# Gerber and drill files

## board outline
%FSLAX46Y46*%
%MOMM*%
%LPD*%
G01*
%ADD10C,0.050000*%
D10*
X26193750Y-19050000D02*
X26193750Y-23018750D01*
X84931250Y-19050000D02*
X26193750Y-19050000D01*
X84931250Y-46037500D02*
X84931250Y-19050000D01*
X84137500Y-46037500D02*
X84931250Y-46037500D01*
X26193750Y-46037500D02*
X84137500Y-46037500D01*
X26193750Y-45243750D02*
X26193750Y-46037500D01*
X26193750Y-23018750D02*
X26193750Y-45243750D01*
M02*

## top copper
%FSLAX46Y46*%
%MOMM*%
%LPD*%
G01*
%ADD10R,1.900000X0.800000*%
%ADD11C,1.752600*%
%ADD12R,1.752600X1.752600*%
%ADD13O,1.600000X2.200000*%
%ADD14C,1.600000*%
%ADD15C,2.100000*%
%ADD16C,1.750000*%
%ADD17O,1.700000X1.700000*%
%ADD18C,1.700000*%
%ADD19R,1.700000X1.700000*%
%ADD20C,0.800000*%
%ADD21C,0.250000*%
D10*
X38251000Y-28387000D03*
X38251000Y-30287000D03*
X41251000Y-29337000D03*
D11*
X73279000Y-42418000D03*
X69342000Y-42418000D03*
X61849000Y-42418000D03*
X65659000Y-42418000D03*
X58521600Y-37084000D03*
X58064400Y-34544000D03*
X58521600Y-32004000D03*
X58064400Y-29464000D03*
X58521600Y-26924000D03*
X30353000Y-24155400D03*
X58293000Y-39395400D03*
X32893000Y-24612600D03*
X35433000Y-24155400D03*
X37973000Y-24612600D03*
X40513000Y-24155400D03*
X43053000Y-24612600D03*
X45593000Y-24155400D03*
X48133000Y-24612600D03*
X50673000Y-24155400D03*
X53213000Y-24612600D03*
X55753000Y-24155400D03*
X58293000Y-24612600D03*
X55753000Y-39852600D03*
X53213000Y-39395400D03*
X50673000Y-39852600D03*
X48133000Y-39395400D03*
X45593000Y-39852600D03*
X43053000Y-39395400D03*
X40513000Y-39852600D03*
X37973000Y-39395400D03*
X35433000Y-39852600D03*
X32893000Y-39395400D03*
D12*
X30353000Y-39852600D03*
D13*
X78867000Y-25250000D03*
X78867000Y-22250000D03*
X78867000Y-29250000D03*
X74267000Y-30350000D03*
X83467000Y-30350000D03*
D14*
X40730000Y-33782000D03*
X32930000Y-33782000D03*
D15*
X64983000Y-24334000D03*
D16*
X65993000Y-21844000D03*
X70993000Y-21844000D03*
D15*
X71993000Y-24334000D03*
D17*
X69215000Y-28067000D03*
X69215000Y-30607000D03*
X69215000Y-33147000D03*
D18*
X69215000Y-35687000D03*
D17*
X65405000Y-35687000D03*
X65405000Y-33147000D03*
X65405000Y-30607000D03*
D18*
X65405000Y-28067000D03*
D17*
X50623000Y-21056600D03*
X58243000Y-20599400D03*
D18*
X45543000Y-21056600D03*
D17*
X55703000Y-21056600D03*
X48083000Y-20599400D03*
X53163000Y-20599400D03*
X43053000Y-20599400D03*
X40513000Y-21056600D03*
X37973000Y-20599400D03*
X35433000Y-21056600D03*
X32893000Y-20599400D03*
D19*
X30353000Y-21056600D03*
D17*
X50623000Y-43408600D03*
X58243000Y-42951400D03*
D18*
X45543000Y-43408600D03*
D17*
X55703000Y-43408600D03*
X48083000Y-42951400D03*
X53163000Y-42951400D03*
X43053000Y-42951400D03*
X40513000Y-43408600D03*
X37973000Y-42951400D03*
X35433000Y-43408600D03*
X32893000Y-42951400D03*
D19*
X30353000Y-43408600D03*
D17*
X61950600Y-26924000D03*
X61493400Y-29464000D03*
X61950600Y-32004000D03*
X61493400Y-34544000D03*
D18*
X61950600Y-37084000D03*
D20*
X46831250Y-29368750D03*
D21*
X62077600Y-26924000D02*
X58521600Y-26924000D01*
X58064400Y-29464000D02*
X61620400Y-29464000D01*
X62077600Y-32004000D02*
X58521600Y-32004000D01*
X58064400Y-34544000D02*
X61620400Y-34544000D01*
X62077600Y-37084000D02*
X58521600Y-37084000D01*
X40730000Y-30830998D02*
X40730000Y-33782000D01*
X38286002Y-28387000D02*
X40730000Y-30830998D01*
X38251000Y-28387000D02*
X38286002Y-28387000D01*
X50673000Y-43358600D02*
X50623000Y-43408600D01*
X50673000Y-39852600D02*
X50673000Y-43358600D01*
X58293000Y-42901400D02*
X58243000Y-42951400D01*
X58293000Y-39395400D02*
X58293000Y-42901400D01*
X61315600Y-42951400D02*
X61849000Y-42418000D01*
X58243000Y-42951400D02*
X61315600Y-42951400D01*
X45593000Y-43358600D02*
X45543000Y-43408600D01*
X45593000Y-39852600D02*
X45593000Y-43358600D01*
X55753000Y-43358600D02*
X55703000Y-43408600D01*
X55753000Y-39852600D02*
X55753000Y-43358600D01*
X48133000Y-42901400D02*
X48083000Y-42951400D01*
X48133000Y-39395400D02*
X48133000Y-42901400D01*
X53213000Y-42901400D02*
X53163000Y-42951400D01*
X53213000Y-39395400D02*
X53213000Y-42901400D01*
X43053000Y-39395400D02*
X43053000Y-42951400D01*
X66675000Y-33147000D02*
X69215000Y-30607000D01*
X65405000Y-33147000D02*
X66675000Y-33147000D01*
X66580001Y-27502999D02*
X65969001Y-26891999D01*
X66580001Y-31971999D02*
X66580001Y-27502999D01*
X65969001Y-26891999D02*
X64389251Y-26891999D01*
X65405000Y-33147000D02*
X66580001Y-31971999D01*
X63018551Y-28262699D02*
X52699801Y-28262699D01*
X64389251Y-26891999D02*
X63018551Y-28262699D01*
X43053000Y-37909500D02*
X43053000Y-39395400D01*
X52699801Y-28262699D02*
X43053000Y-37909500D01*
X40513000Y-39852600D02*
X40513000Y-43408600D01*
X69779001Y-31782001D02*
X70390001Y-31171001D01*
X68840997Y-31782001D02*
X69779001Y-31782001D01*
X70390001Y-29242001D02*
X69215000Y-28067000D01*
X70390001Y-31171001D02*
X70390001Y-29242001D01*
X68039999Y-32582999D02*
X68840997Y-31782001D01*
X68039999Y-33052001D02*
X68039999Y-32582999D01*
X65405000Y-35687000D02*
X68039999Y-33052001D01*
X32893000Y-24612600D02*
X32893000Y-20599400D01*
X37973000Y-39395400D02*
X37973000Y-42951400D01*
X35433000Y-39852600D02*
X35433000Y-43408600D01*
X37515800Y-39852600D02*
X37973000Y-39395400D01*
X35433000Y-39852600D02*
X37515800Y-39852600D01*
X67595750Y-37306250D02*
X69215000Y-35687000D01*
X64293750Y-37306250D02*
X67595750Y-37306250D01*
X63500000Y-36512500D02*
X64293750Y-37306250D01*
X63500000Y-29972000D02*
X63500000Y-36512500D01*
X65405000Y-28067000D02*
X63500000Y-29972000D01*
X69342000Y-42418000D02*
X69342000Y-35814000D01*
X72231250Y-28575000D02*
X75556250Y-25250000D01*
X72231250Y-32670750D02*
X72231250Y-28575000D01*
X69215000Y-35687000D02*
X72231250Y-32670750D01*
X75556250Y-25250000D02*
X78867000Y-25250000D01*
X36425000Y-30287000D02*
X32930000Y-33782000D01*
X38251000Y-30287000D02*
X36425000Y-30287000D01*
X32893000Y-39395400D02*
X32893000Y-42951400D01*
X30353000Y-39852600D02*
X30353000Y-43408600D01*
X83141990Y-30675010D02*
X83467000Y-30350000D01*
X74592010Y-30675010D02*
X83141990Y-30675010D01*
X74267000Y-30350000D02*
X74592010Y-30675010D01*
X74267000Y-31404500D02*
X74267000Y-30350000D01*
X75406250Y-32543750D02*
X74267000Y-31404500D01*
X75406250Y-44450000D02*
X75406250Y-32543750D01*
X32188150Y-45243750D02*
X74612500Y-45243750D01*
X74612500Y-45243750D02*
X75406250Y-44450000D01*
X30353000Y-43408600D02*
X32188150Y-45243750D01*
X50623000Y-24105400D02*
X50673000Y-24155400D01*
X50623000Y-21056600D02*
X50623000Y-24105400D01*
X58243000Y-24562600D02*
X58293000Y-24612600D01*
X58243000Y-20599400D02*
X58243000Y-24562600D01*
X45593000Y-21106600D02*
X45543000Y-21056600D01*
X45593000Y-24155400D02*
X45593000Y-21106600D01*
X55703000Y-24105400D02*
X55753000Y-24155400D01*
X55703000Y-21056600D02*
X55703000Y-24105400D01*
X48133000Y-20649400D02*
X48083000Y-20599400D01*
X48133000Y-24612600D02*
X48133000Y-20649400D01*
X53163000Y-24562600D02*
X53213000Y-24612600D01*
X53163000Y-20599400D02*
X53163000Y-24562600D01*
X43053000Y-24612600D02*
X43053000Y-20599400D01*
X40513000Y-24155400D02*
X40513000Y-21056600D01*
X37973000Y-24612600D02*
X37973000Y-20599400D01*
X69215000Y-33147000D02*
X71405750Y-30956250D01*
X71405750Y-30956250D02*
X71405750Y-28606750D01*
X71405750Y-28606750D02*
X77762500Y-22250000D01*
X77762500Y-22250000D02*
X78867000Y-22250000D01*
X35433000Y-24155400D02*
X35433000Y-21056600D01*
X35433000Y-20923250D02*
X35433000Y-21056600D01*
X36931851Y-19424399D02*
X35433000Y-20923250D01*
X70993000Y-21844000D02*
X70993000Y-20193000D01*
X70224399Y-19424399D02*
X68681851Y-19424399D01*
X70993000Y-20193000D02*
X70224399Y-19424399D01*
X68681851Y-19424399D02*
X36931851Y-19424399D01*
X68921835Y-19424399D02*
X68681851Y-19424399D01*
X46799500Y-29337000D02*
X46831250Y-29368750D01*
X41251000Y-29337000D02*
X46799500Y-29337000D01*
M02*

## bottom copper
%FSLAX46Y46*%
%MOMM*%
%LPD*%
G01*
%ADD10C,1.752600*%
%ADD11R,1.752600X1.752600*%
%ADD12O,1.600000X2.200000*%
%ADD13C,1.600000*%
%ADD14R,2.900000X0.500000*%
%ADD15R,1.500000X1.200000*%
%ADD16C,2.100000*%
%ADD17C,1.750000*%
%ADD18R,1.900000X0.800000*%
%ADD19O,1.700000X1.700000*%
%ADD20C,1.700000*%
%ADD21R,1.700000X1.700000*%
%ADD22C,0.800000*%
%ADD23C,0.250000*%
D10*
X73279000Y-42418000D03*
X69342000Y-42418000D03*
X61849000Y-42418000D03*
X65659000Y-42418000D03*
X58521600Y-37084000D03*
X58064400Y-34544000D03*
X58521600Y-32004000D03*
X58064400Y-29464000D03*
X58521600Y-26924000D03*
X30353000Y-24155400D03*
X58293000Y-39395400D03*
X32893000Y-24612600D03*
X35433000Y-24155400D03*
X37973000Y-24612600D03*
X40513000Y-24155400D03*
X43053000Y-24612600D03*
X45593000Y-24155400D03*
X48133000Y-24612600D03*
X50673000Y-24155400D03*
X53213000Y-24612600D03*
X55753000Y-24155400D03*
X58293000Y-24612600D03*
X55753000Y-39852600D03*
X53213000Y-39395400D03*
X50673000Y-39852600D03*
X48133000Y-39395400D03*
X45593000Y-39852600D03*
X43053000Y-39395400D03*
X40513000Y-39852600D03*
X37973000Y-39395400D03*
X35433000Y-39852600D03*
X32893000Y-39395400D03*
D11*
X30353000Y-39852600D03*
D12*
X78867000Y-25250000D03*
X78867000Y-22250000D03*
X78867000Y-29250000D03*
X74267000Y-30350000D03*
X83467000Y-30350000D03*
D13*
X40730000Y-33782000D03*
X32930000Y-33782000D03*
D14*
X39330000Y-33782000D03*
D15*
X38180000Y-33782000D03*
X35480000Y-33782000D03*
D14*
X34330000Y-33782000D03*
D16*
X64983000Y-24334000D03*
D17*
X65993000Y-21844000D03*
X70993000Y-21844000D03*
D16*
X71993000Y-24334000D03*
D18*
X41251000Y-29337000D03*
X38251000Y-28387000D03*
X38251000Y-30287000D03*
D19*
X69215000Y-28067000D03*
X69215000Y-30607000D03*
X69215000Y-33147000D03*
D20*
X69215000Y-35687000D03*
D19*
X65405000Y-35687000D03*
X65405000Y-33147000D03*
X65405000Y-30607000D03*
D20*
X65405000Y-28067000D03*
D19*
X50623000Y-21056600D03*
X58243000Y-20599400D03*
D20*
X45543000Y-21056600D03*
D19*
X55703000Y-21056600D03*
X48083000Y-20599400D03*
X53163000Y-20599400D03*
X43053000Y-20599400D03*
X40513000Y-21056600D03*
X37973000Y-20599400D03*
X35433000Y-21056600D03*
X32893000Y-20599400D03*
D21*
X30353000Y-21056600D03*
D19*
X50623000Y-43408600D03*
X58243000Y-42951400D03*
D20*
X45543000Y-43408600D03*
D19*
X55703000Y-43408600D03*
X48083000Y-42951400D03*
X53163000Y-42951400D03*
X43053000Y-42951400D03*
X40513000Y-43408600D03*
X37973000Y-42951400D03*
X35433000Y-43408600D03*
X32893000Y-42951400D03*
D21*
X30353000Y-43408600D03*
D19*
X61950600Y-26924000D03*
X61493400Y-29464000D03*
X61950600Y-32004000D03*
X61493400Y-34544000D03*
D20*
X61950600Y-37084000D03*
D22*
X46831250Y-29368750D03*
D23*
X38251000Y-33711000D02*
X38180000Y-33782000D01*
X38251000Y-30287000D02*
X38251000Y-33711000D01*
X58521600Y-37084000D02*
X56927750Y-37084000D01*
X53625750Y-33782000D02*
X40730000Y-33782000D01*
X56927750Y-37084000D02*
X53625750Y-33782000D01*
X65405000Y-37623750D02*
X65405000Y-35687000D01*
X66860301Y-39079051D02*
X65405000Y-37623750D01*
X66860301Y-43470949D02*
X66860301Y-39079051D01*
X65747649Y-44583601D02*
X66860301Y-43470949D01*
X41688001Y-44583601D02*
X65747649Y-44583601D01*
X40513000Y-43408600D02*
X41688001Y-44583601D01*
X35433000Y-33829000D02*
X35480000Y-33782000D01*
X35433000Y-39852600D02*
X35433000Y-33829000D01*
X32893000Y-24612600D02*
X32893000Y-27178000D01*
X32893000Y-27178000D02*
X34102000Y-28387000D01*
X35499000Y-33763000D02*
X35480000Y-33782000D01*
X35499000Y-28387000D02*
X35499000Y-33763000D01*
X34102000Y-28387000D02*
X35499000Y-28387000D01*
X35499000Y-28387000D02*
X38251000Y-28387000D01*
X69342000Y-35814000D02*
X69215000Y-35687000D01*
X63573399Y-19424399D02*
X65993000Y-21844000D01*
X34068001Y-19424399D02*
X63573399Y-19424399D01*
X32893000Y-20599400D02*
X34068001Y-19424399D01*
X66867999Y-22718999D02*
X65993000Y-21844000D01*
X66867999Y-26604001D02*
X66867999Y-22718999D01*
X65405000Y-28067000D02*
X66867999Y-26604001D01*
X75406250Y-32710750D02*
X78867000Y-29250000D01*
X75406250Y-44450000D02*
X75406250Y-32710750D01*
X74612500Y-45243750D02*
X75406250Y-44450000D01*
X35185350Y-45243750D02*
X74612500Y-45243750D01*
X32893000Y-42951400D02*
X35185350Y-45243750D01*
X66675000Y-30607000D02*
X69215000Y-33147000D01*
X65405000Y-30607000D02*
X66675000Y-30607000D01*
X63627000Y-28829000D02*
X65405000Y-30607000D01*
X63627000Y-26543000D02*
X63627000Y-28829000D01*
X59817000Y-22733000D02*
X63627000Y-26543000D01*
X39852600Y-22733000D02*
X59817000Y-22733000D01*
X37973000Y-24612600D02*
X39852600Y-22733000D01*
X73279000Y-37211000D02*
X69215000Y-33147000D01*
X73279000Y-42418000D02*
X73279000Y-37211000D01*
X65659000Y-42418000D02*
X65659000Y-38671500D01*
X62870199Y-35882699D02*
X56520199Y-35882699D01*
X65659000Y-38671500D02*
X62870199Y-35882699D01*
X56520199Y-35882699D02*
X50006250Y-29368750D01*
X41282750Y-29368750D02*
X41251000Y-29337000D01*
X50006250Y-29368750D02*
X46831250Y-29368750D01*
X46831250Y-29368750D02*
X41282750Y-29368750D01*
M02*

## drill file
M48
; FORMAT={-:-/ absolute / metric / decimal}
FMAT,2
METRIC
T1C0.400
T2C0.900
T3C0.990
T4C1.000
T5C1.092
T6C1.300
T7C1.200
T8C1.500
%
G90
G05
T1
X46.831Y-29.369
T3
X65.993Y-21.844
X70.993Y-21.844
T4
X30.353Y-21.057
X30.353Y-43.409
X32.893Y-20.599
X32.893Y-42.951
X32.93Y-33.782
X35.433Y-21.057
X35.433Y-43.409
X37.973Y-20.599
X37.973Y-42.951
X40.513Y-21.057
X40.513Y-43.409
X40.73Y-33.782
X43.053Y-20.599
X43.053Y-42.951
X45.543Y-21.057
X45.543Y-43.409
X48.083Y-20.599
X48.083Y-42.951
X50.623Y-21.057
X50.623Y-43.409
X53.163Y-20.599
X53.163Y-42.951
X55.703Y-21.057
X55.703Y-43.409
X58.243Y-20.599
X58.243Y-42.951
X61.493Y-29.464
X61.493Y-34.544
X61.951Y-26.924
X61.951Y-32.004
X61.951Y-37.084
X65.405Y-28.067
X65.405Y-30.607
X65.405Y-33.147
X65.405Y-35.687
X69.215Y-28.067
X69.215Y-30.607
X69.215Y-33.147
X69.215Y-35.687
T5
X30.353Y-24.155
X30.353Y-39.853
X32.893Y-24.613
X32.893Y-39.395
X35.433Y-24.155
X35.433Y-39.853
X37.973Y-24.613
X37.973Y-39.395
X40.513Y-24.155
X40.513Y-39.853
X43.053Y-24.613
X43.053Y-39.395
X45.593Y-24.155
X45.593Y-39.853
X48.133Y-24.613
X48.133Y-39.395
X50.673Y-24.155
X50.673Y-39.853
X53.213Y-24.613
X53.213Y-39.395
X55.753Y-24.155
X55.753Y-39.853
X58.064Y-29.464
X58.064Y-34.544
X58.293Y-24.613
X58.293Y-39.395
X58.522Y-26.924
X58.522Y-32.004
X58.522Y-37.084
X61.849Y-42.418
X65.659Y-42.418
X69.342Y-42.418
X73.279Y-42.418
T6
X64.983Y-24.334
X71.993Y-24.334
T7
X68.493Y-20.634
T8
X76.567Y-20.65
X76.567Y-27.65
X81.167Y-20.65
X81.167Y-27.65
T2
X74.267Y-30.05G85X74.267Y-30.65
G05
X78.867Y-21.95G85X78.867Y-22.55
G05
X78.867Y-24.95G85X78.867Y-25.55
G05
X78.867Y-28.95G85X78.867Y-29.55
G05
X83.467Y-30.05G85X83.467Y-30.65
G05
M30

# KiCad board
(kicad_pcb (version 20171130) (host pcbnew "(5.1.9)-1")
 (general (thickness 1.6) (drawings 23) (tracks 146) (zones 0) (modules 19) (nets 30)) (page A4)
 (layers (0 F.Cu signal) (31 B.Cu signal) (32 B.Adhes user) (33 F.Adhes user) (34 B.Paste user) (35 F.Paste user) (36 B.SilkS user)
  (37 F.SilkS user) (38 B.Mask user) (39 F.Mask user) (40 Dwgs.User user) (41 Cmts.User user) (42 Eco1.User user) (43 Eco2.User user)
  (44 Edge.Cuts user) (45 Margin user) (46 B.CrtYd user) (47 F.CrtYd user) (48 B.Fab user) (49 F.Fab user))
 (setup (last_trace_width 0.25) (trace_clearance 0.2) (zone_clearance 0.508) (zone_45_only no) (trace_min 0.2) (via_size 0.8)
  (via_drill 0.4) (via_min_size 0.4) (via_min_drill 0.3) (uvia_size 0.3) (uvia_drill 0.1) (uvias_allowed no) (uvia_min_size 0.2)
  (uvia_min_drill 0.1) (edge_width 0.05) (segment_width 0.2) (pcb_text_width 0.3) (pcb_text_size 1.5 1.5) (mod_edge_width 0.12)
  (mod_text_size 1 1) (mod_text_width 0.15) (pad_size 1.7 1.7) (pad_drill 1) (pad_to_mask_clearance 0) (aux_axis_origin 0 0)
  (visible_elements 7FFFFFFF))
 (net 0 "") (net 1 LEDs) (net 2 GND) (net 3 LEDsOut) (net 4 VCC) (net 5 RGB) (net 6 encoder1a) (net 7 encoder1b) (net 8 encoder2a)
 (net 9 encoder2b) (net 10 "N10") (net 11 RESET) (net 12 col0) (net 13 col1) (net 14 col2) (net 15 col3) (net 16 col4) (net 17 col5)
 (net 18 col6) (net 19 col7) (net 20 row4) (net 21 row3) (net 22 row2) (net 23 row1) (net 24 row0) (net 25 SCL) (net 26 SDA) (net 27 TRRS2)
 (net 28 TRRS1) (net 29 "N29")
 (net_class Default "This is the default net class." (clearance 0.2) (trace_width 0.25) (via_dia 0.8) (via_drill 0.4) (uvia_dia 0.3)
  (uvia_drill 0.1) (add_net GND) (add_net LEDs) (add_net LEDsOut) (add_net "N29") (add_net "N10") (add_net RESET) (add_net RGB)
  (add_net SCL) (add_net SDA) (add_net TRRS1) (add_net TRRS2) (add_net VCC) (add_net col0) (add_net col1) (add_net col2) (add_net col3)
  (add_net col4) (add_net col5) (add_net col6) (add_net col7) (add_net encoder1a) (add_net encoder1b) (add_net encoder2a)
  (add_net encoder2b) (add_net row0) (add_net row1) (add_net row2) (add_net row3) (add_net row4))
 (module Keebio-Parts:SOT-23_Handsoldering (layer F.Cu) (at 39.751 29.337)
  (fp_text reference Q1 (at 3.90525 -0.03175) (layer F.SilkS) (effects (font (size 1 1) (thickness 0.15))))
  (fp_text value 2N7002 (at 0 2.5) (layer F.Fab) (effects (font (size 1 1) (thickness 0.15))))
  (pad 1 smd rect (at -1.5 -0.95) (size 1.9 0.8) (layers F.Cu F.Paste F.Mask) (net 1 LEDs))
  (pad 2 smd rect (at -1.5 0.95) (size 1.9 0.8) (layers F.Cu F.Paste F.Mask) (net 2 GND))
  (pad 3 smd rect (at 1.5 0) (size 1.9 0.8) (layers F.Cu F.Paste F.Mask) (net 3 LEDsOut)))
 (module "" (layer F.Cu) (at 73.914 49.149)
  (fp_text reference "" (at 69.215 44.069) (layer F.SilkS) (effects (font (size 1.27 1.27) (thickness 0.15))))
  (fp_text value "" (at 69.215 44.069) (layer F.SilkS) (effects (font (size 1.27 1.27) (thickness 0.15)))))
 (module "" (layer F.Cu) (at 69.215 44.069)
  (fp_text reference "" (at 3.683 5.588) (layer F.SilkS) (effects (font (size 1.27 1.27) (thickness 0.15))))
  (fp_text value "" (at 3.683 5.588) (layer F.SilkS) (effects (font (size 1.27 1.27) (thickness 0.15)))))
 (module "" (layer F.Cu) (at 3.683 5.588)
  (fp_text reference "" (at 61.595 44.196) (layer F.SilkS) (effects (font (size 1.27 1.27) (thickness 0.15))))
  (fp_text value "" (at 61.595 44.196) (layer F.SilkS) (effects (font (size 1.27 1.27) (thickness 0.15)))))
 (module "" (layer F.Cu) (at 61.595 44.196)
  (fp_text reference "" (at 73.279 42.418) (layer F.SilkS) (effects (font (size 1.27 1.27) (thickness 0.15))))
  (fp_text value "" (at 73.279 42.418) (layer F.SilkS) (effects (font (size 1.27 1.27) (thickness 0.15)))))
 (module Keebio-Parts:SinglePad (layer F.Cu) (at 73.279 42.418)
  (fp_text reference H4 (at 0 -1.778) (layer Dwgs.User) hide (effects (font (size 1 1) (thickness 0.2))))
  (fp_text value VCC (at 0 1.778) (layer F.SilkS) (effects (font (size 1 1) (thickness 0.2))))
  (pad 1 thru_hole circle (at 0 0 270) (size 1.7526 1.7526) (drill 1.0922) (layers *.Cu *.SilkS *.Mask) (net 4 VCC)))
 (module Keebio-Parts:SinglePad (layer F.Cu) (at 69.342 42.418)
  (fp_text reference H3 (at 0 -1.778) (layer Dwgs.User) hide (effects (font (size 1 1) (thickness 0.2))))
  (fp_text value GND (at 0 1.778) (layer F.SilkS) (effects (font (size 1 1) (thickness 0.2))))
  (pad 1 thru_hole circle (at 0 0 270) (size 1.7526 1.7526) (drill 1.0922) (layers *.Cu *.SilkS *.Mask) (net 2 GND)))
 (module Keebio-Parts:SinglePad (layer F.Cu) (at 61.849 42.418)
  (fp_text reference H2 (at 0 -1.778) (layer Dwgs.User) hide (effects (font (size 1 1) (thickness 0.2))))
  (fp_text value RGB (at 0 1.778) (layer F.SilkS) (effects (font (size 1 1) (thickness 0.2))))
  (pad 1 thru_hole circle (at 0 0 270) (size 1.7526 1.7526) (drill 1.0922) (layers *.Cu *.SilkS *.Mask) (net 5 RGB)))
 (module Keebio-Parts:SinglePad (layer F.Cu) (at 65.659 42.418)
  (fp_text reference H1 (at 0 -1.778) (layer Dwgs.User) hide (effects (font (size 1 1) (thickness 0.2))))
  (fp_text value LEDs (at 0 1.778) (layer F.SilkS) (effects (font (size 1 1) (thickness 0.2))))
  (pad 1 thru_hole circle (at 0 0 270) (size 1.7526 1.7526) (drill 1.0922) (layers *.Cu *.SilkS *.Mask) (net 3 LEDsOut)))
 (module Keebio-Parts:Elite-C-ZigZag (layer F.Cu) (at 44.323 32.004)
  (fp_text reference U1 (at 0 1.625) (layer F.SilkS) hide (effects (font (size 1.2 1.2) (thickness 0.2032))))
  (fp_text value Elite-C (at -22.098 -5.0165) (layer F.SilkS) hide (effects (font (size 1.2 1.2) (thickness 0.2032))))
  (pad 25 thru_hole circle (at 14.1986 5.08) (size 1.7526 1.7526) (drill 1.0922) (layers *.Cu *.SilkS *.Mask) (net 1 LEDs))
  (pad 26 thru_hole circle (at 13.7414 2.54) (size 1.7526 1.7526) (drill 1.0922) (layers *.Cu *.SilkS *.Mask) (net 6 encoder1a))
  (pad 27 thru_hole circle (at 14.1986 0) (size 1.7526 1.7526) (drill 1.0922) (layers *.Cu *.SilkS *.Mask) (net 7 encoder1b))
  (pad 28 thru_hole circle (at 13.7414 -2.54) (size 1.7526 1.7526) (drill 1.0922) (layers *.Cu *.SilkS *.Mask) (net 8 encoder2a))
  (pad 29 thru_hole circle (at 14.1986 -5.08) (size 1.7526 1.7526) (drill 1.0922) (layers *.Cu *.SilkS *.Mask) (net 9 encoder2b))
  (pad 24 thru_hole circle (at -13.97 -7.8486) (size 1.7526 1.7526) (drill 1.0922) (layers *.Cu *.SilkS *.Mask) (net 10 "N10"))
  (pad 12 thru_hole circle (at 13.97 7.3914) (size 1.7526 1.7526) (drill 1.0922) (layers *.Cu *.SilkS *.Mask) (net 5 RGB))
  (pad 23 thru_hole circle (at -11.43 -7.3914) (size 1.7526 1.7526) (drill 1.0922) (layers *.Cu *.SilkS *.Mask) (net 2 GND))
  (pad 22 thru_hole circle (at -8.89 -7.8486) (size 1.7526 1.7526) (drill 1.0922) (layers *.Cu *.SilkS *.Mask) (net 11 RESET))
  (pad 21 thru_hole circle (at -6.35 -7.3914) (size 1.7526 1.7526) (drill 1.0922) (layers *.Cu *.SilkS *.Mask) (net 4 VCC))
  (pad 20 thru_hole circle (at -3.81 -7.8486) (size 1.7526 1.7526) (drill 1.0922) (layers *.Cu *.SilkS *.Mask) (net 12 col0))
  (pad 19 thru_hole circle (at -1.27 -7.3914) (size 1.7526 1.7526) (drill 1.0922) (layers *.Cu *.SilkS *.Mask) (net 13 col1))
  (pad 18 thru_hole circle (at 1.27 -7.8486) (size 1.7526 1.7526) (drill 1.0922) (layers *.Cu *.SilkS *.Mask) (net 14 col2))
  (pad 17 thru_hole circle (at 3.81 -7.3914) (size 1.7526 1.7526) (drill 1.0922) (layers *.Cu *.SilkS *.Mask) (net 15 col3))
  (pad 16 thru_hole circle (at 6.35 -7.8486) (size 1.7526 1.7526) (drill 1.0922) (layers *.Cu *.SilkS *.Mask) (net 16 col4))
  (pad 15 thru_hole circle (at 8.89 -7.3914) (size 1.7526 1.7526) (drill 1.0922) (layers *.Cu *.SilkS *.Mask) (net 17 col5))
  (pad 14 thru_hole circle (at 11.43 -7.8486) (size 1.7526 1.7526) (drill 1.0922) (layers *.Cu *.SilkS *.Mask) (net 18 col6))
  (pad 13 thru_hole circle (at 13.97 -7.3914) (size 1.7526 1.7526) (drill 1.0922) (layers *.Cu *.SilkS *.Mask) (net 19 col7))
  (pad 11 thru_hole circle (at 11.43 7.8486) (size 1.7526 1.7526) (drill 1.0922) (layers *.Cu *.SilkS *.Mask) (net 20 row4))
  (pad 10 thru_hole circle (at 8.89 7.3914) (size 1.7526 1.7526) (drill 1.0922) (layers *.Cu *.SilkS *.Mask) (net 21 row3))
  (pad 9 thru_hole circle (at 6.35 7.8486) (size 1.7526 1.7526) (drill 1.0922) (layers *.Cu *.SilkS *.Mask) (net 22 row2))
  (pad 8 thru_hole circle (at 3.81 7.3914) (size 1.7526 1.7526) (drill 1.0922) (layers *.Cu *.SilkS *.Mask) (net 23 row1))
  (pad 7 thru_hole circle (at 1.27 7.8486) (size 1.7526 1.7526) (drill 1.0922) (layers *.Cu *.SilkS *.Mask) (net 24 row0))
  (pad 6 thru_hole circle (at -1.27 7.3914) (size 1.7526 1.7526) (drill 1.0922) (layers *.Cu *.SilkS *.Mask) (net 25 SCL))
  (pad 5 thru_hole circle (at -3.81 7.8486) (size 1.7526 1.7526) (drill 1.0922) (layers *.Cu *.SilkS *.Mask) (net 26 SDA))
  (pad 4 thru_hole circle (at -6.35 7.3914) (size 1.7526 1.7526) (drill 1.0922) (layers *.Cu *.SilkS *.Mask) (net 2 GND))
  (pad 3 thru_hole circle (at -8.89 7.8486) (size 1.7526 1.7526) (drill 1.0922) (layers *.Cu *.SilkS *.Mask) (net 2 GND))
  (pad 2 thru_hole circle (at -11.43 7.3914) (size 1.7526 1.7526) (drill 1.0922) (layers *.Cu *.SilkS *.Mask) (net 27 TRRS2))
  (pad 1 thru_hole rect (at -13.97 7.8486) (size 1.7526 1.7526) (drill 1.0922) (layers *.Cu *.SilkS *.Mask) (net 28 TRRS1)))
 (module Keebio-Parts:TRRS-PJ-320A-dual (layer F.Cu) (at 78.867 19.05)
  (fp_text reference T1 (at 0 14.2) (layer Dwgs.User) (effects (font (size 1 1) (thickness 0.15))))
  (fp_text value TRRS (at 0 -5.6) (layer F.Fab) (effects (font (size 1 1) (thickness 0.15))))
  (pad 3 thru_hole oval (at 0 6.2) (size 1.6 2.2) (drill oval 0.9 1.5) (layers *.Cu *.Mask) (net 2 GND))
  (pad "" np_thru_hole circle (at -2.3 1.6) (size 1.5 1.5) (drill 1.5) (layers *.Cu *.Mask))
  (pad "" np_thru_hole circle (at -2.3 8.6) (size 1.5 1.5) (drill 1.5) (layers *.Cu *.Mask))
  (pad 4 thru_hole oval (at 0 3.2) (size 1.6 2.2) (drill oval 0.9 1.5) (layers *.Cu *.Mask) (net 4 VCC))
  (pad 2 thru_hole oval (at 0 10.2) (size 1.6 2.2) (drill oval 0.9 1.5) (layers *.Cu *.Mask) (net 27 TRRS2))
  (pad 1 thru_hole oval (at -4.6 11.3) (size 1.6 2.2) (drill oval 0.9 1.5) (layers *.Cu *.Mask) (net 28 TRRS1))
  (pad 1 thru_hole oval (at 4.6 11.3) (size 1.6 2.2) (drill oval 0.9 1.5) (layers *.Cu *.Mask) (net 28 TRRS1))
  (pad "" np_thru_hole circle (at 2.3 1.6) (size 1.5 1.5) (drill 1.5) (layers *.Cu *.Mask))
  (pad "" np_thru_hole circle (at 2.3 8.6) (size 1.5 1.5) (drill 1.5) (layers *.Cu *.Mask)))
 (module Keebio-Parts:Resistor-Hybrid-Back (layer F.Cu) (at 36.83 33.782)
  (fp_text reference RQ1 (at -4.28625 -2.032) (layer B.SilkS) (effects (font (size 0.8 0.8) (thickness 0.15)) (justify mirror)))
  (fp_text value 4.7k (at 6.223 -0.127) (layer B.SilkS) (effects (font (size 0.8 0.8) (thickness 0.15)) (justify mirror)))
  (pad 1 thru_hole circle (at 3.9 0) (size 1.6 1.6) (drill 1) (layers *.Cu *.Mask) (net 1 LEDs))
  (pad 2 thru_hole circle (at -3.9 0) (size 1.6 1.6) (drill 1) (layers *.Cu *.Mask F.SilkS) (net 2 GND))
  (pad 1 smd rect (at 2.5 0) (size 2.9 0.5) (layers B.Cu) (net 1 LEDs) (solder_mask_margin -999))
  (pad 1 smd rect (at 1.35 0) (size 1.5 1.2) (layers B.Cu B.Paste B.Mask) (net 1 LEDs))
  (pad 2 smd rect (at -1.35 0) (size 1.5 1.2) (layers B.Cu B.Paste B.Mask) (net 2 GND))
  (pad 2 smd rect (at -2.5 0) (size 2.9 0.5) (layers B.Cu) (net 2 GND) (solder_mask_margin -999)))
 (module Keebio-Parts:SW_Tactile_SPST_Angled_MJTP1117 (layer B.Cu) (at 70.993 21.844 180)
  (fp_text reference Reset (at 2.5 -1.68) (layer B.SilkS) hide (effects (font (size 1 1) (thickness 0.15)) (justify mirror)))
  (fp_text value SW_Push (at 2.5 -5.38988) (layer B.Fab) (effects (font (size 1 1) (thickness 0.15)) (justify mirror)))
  (pad "" thru_hole circle (at 6.01 -2.49 180) (size 2.1 2.1) (drill 1.3) (layers *.Cu *.Mask))
  (pad 2 thru_hole circle (at 5 0 180) (size 1.75 1.75) (drill 0.99) (layers *.Cu *.Mask) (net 2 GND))
  (pad 1 thru_hole circle (at 0 0 180) (size 1.75 1.75) (drill 0.99) (layers *.Cu *.Mask) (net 11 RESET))
  (pad "" thru_hole circle (at -1 -2.49 180) (size 2.1 2.1) (drill 1.3) (layers *.Cu *.Mask))
  (pad "" np_thru_hole circle (at 2.5 1.21 180) (size 1.2 1.2) (drill 1.2) (layers *.Cu *.Mask)))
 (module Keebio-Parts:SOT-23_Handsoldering (layer B.Cu) (at 39.751 29.337)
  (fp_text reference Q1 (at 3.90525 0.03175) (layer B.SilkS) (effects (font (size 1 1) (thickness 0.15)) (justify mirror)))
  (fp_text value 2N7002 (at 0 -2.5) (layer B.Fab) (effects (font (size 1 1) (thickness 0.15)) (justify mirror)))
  (pad 3 smd rect (at 1.5 0) (size 1.9 0.8) (layers B.Cu B.Paste B.Mask) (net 3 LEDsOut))
  (pad 2 smd rect (at -1.5 -0.95) (size 1.9 0.8) (layers B.Cu B.Paste B.Mask) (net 2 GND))
  (pad 1 smd rect (at -1.5 0.95) (size 1.9 0.8) (layers B.Cu B.Paste B.Mask) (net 1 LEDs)))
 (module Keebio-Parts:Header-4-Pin (layer F.Cu) (at 69.215 35.687 180)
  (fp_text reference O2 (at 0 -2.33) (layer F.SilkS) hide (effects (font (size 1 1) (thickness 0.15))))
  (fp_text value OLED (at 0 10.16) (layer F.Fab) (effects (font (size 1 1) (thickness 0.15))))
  (pad 4 thru_hole oval (at 0 7.62 180) (size 1.7 1.7) (drill 1) (layers *.Cu *.Mask) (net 26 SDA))
  (pad 3 thru_hole oval (at 0 5.08 180) (size 1.7 1.7) (drill 1) (layers *.Cu *.Mask) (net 25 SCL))
  (pad 2 thru_hole oval (at 0 2.54 180) (size 1.7 1.7) (drill 1) (layers *.Cu *.Mask) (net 4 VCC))
  (pad 1 thru_hole circle (at 0 0 180) (size 1.7 1.7) (drill 1) (layers *.Cu *.Mask) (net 2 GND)))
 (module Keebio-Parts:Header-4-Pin (layer F.Cu) (at 65.405 28.067)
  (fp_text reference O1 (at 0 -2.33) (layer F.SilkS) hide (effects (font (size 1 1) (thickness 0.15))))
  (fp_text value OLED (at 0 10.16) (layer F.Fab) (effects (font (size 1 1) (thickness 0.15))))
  (pad 4 thru_hole oval (at 0 7.62) (size 1.7 1.7) (drill 1) (layers *.Cu *.Mask) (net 26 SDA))
  (pad 3 thru_hole oval (at 0 5.08) (size 1.7 1.7) (drill 1) (layers *.Cu *.Mask) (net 25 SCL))
  (pad 2 thru_hole oval (at 0 2.54) (size 1.7 1.7) (drill 1) (layers *.Cu *.Mask) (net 4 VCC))
  (pad 1 thru_hole circle (at 0 0) (size 1.7 1.7) (drill 1) (layers *.Cu *.Mask) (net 2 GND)))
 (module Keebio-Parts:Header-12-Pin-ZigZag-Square (layer F.Cu) (at 30.353 20.828 90)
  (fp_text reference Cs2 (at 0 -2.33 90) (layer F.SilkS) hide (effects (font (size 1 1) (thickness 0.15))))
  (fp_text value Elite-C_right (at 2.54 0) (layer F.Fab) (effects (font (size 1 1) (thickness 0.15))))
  (pad 9 thru_hole oval (at -0.2286 20.27 90) (size 1.7 1.7) (drill 1) (layers *.Cu *.Mask) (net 16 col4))
  (pad 12 thru_hole oval (at 0.2286 27.89 90) (size 1.7 1.7) (drill 1) (layers *.Cu *.Mask) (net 19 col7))
  (pad 7 thru_hole circle (at -0.2286 15.19 90) (size 1.7 1.7) (drill 1) (layers *.Cu *.Mask) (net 14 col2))
  (pad 11 thru_hole oval (at -0.2286 25.35 90) (size 1.7 1.7) (drill 1) (layers *.Cu *.Mask) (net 18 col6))
  (pad 8 thru_hole oval (at 0.2286 17.73 90) (size 1.7 1.7) (drill 1) (layers *.Cu *.Mask) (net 15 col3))
  (pad 10 thru_hole oval (at 0.2286 22.81 90) (size 1.7 1.7) (drill 1) (layers *.Cu *.Mask) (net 17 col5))
  (pad 6 thru_hole oval (at 0.2286 12.7 90) (size 1.7 1.7) (drill 1) (layers *.Cu *.Mask) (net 13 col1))
  (pad 5 thru_hole oval (at -0.2286 10.16 90) (size 1.7 1.7) (drill 1) (layers *.Cu *.Mask) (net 12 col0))
  (pad 4 thru_hole oval (at 0.2286 7.62 90) (size 1.7 1.7) (drill 1) (layers *.Cu *.Mask) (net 4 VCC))
  (pad 3 thru_hole oval (at -0.2286 5.08 90) (size 1.7 1.7) (drill 1) (layers *.Cu *.Mask) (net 11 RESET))
  (pad 2 thru_hole oval (at 0.2286 2.54 90) (size 1.7 1.7) (drill 1) (layers *.Cu *.Mask) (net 2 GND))
  (pad 1 thru_hole rect (at -0.2286 0 90) (size 1.7 1.7) (drill 1) (layers *.Cu *.Mask) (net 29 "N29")))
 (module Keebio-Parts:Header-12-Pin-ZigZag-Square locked (layer F.Cu) (at 30.353 43.18 90)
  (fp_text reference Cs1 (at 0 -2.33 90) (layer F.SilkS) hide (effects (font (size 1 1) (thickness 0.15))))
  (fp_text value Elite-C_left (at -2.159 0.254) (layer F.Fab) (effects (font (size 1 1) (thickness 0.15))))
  (pad 9 thru_hole oval (at -0.2286 20.27 90) (size 1.7 1.7) (drill 1) (layers *.Cu *.Mask) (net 22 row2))
  (pad 12 thru_hole oval (at 0.2286 27.89 90) (size 1.7 1.7) (drill 1) (layers *.Cu *.Mask) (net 5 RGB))
  (pad 7 thru_hole circle (at -0.2286 15.19 90) (size 1.7 1.7) (drill 1) (layers *.Cu *.Mask) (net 24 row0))
  (pad 11 thru_hole oval (at -0.2286 25.35 90) (size 1.7 1.7) (drill 1) (layers *.Cu *.Mask) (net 20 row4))
  (pad 8 thru_hole oval (at 0.2286 17.73 90) (size 1.7 1.7) (drill 1) (layers *.Cu *.Mask) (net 23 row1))
  (pad 10 thru_hole oval (at 0.2286 22.81 90) (size 1.7 1.7) (drill 1) (layers *.Cu *.Mask) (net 21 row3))
  (pad 6 thru_hole oval (at 0.2286 12.7 90) (size 1.7 1.7) (drill 1) (layers *.Cu *.Mask) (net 25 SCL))
  (pad 5 thru_hole oval (at -0.2286 10.16 90) (size 1.7 1.7) (drill 1) (layers *.Cu *.Mask) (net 26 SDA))
  (pad 4 thru_hole oval (at 0.2286 7.62 90) (size 1.7 1.7) (drill 1) (layers *.Cu *.Mask) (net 2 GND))
  (pad 3 thru_hole oval (at -0.2286 5.08 90) (size 1.7 1.7) (drill 1) (layers *.Cu *.Mask) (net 2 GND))
  (pad 2 thru_hole oval (at 0.2286 2.54 90) (size 1.7 1.7) (drill 1) (layers *.Cu *.Mask) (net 27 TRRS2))
  (pad 1 thru_hole rect (at -0.2286 0 90) (size 1.7 1.7) (drill 1) (layers *.Cu *.Mask) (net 28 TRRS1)))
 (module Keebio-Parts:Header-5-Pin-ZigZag (layer F.Cu) (at 61.722 37.084 180)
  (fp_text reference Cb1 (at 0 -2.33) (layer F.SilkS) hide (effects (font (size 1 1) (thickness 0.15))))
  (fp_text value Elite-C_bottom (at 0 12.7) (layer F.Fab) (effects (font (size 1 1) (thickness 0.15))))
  (pad 5 thru_hole oval (at -0.2286 10.16 180) (size 1.7 1.7) (drill 1) (layers *.Cu *.Mask) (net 9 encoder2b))
  (pad 4 thru_hole oval (at 0.2286 7.62 180) (size 1.7 1.7) (drill 1) (layers *.Cu *.Mask) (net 8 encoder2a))
  (pad 3 thru_hole oval (at -0.2286 5.08 180) (size 1.7 1.7) (drill 1) (layers *.Cu *.Mask) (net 7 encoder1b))
  (pad 2 thru_hole oval (at 0.2286 2.54 180) (size 1.7 1.7) (drill 1) (layers *.Cu *.Mask) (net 6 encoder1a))
  (pad 1 thru_hole circle (at -0.2286 0 180) (size 1.7 1.7) (drill 1) (layers *.Cu *.Mask) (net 1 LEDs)))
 (gr_line (start 26.19375 19.05) (end 26.19375 23.01875) (layer Edge.Cuts) (width 0.05))
 (gr_line (start 84.93125 19.05) (end 26.19375 19.05) (layer Edge.Cuts) (width 0.05))
 (gr_line (start 84.93125 46.0375) (end 84.93125 19.05) (layer Edge.Cuts) (width 0.05))
 (gr_line (start 84.1375 46.0375) (end 84.93125 46.0375) (layer Edge.Cuts) (width 0.05))
 (gr_line (start 26.19375 46.0375) (end 84.1375 46.0375) (layer Edge.Cuts) (width 0.05))
 (gr_line (start 26.19375 45.24375) (end 26.19375 46.0375) (layer Edge.Cuts) (width 0.05))
 (gr_line (start 26.19375 23.01875) (end 26.19375 45.24375) (layer Edge.Cuts) (width 0.05))
 (segment (start 62.0776 26.924) (end 58.5216 26.924) (width 0.25) (layer F.Cu) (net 9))
 (segment (start 58.0644 29.464) (end 61.6204 29.464) (width 0.25) (layer F.Cu) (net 8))
 (segment (start 62.0776 32.004) (end 58.5216 32.004) (width 0.25) (layer F.Cu) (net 7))
 (segment (start 58.0644 34.544) (end 61.6204 34.544) (width 0.25) (layer F.Cu) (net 6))
 (segment (start 62.0776 37.084) (end 58.5216 37.084) (width 0.25) (layer F.Cu) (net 1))
 (segment (start 38.251 33.711) (end 38.18 33.782) (width 0.25) (layer B.Cu) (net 1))
 (segment (start 38.251 30.287) (end 38.251 33.711) (width 0.25) (layer B.Cu) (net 1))
 (segment (start 58.5216 37.084) (end 56.92775 37.084) (width 0.25) (layer B.Cu) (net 1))
 (segment (start 53.62575 33.782) (end 40.73 33.782) (width 0.25) (layer B.Cu) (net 1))
 (segment (start 56.92775 37.084) (end 53.62575 33.782) (width 0.25) (layer B.Cu) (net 1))
 (segment (start 40.73 30.830998) (end 40.73 33.782) (width 0.25) (layer F.Cu) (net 1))
 (segment (start 38.286002 28.387) (end 40.73 30.830998) (width 0.25) (layer F.Cu) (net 1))
 (segment (start 38.251 28.387) (end 38.286002 28.387) (width 0.25) (layer F.Cu) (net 1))
 (segment (start 50.673 43.3586) (end 50.623 43.4086) (width 0.25) (layer F.Cu) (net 22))
 (segment (start 50.673 39.8526) (end 50.673 43.3586) (width 0.25) (layer F.Cu) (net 22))
 (segment (start 58.293 42.9014) (end 58.243 42.9514) (width 0.25) (layer F.Cu) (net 5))
 (segment (start 58.293 39.3954) (end 58.293 42.9014) (width 0.25) (layer F.Cu) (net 5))
 (segment (start 61.3156 42.9514) (end 61.849 42.418) (width 0.25) (layer F.Cu) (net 5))
 (segment (start 58.243 42.9514) (end 61.3156 42.9514) (width 0.25) (layer F.Cu) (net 5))
 (segment (start 45.593 43.3586) (end 45.543 43.4086) (width 0.25) (layer F.Cu) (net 24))
 (segment (start 45.593 39.8526) (end 45.593 43.3586) (width 0.25) (layer F.Cu) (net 24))
 (segment (start 55.753 43.3586) (end 55.703 43.4086) (width 0.25) (layer F.Cu) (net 20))
 (segment (start 55.753 39.8526) (end 55.753 43.3586) (width 0.25) (layer F.Cu) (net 20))
 (segment (start 48.133 42.9014) (end 48.083 42.9514) (width 0.25) (layer F.Cu) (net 23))
 (segment (start 48.133 39.3954) (end 48.133 42.9014) (width 0.25) (layer F.Cu) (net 23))
 (segment (start 53.213 42.9014) (end 53.163 42.9514) (width 0.25) (layer F.Cu) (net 21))
 (segment (start 53.213 39.3954) (end 53.213 42.9014) (width 0.25) (layer F.Cu) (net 21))
 (segment (start 43.053 39.3954) (end 43.053 42.9514) (width 0.25) (layer F.Cu) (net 25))
 (segment (start 66.675 33.147) (end 69.215 30.607) (width 0.25) (layer F.Cu) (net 25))
 (segment (start 65.405 33.147) (end 66.675 33.147) (width 0.25) (layer F.Cu) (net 25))
 (segment (start 66.580001 27.502999) (end 65.969001 26.891999) (width 0.25) (layer F.Cu) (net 25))
 (segment (start 66.580001 31.971999) (end 66.580001 27.502999) (width 0.25) (layer F.Cu) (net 25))
 (segment (start 65.969001 26.891999) (end 64.389251 26.891999) (width 0.25) (layer F.Cu) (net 25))
 (segment (start 65.405 33.147) (end 66.580001 31.971999) (width 0.25) (layer F.Cu) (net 25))
 (segment (start 63.018551 28.262699) (end 52.699801 28.262699) (width 0.25) (layer F.Cu) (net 25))
 (segment (start 64.389251 26.891999) (end 63.018551 28.262699) (width 0.25) (layer F.Cu) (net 25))
 (segment (start 43.053 37.9095) (end 43.053 39.3954) (width 0.25) (layer F.Cu) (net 25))
 (segment (start 52.699801 28.262699) (end 43.053 37.9095) (width 0.25) (layer F.Cu) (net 25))
 (segment (start 40.513 39.8526) (end 40.513 43.4086) (width 0.25) (layer F.Cu) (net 26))
 (segment (start 69.779001 31.782001) (end 70.390001 31.171001) (width 0.25) (layer F.Cu) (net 26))
 (segment (start 68.840997 31.782001) (end 69.779001 31.782001) (width 0.25) (layer F.Cu) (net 26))
 (segment (start 70.390001 29.242001) (end 69.215 28.067) (width 0.25) (layer F.Cu) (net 26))
 (segment (start 70.390001 31.171001) (end 70.390001 29.242001) (width 0.25) (layer F.Cu) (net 26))
 (segment (start 68.039999 32.582999) (end 68.840997 31.782001) (width 0.25) (layer F.Cu) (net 26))
 (segment (start 68.039999 33.052001) (end 68.039999 32.582999) (width 0.25) (layer F.Cu) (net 26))
 (segment (start 65.405 35.687) (end 68.039999 33.052001) (width 0.25) (layer F.Cu) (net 26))
 (segment (start 65.405 37.62375) (end 65.405 35.687) (width 0.25) (layer B.Cu) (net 26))
 (segment (start 66.860301 39.079051) (end 65.405 37.62375) (width 0.25) (layer B.Cu) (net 26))
 (segment (start 66.860301 43.470949) (end 66.860301 39.079051) (width 0.25) (layer B.Cu) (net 26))
 (segment (start 65.747649 44.583601) (end 66.860301 43.470949) (width 0.25) (layer B.Cu) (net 26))
 (segment (start 41.688001 44.583601) (end 65.747649 44.583601) (width 0.25) (layer B.Cu) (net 26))
 (segment (start 40.513 43.4086) (end 41.688001 44.583601) (width 0.25) (layer B.Cu) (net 26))
 (segment (start 32.893 24.6126) (end 32.893 20.5994) (width 0.25) (layer F.Cu) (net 2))
 (segment (start 37.973 39.3954) (end 37.973 42.9514) (width 0.25) (layer F.Cu) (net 2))
 (segment (start 35.433 39.8526) (end 35.433 43.4086) (width 0.25) (layer F.Cu) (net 2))
 (segment (start 37.5158 39.8526) (end 37.973 39.3954) (width 0.25) (layer F.Cu) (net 2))
 (segment (start 35.433 39.8526) (end 37.5158 39.8526) (width 0.25) (layer F.Cu) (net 2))
 (segment (start 35.433 33.829) (end 35.48 33.782) (width 0.25) (layer B.Cu) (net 2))
 (segment (start 35.433 39.8526) (end 35.433 33.829) (width 0.25) (layer B.Cu) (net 2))
 (segment (start 32.893 24.6126) (end 32.893 27.178) (width 0.25) (layer B.Cu) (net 2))
 (segment (start 32.893 27.178) (end 34.102 28.387) (width 0.25) (layer B.Cu) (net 2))
 (segment (start 35.499 33.763) (end 35.48 33.782) (width 0.25) (layer B.Cu) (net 2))
 (segment (start 35.499 28.387) (end 35.499 33.763) (width 0.25) (layer B.Cu) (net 2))
 (segment (start 34.102 28.387) (end 35.499 28.387) (width 0.25) (layer B.Cu) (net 2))
 (segment (start 35.499 28.387) (end 38.251 28.387) (width 0.25) (layer B.Cu) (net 2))
 (segment (start 67.59575 37.30625) (end 69.215 35.687) (width 0.25) (layer F.Cu) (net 2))
 (segment (start 64.29375 37.30625) (end 67.59575 37.30625) (width 0.25) (layer F.Cu) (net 2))
 (segment (start 63.5 36.5125) (end 64.29375 37.30625) (width 0.25) (layer F.Cu) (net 2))
 (segment (start 63.5 29.972) (end 63.5 36.5125) (width 0.25) (layer F.Cu) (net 2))
 (segment (start 65.405 28.067) (end 63.5 29.972) (width 0.25) (layer F.Cu) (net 2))
 (segment (start 69.342 35.814) (end 69.215 35.687) (width 0.25) (layer B.Cu) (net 2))
 (segment (start 69.342 42.418) (end 69.342 35.814) (width 0.25) (layer F.Cu) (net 2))
 (segment (start 72.23125 28.575) (end 75.55625 25.25) (width 0.25) (layer F.Cu) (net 2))
 (segment (start 72.23125 32.67075) (end 72.23125 28.575) (width 0.25) (layer F.Cu) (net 2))
 (segment (start 69.215 35.687) (end 72.23125 32.67075) (width 0.25) (layer F.Cu) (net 2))
 (segment (start 63.573399 19.424399) (end 65.993 21.844) (width 0.25) (layer B.Cu) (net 2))
 (segment (start 34.068001 19.424399) (end 63.573399 19.424399) (width 0.25) (layer B.Cu) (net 2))
 (segment (start 32.893 20.5994) (end 34.068001 19.424399) (width 0.25) (layer B.Cu) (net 2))
 (segment (start 66.867999 22.718999) (end 65.993 21.844) (width 0.25) (layer B.Cu) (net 2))
 (segment (start 66.867999 26.604001) (end 66.867999 22.718999) (width 0.25) (layer B.Cu) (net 2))
 (segment (start 65.405 28.067) (end 66.867999 26.604001) (width 0.25) (layer B.Cu) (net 2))
 (segment (start 75.55625 25.25) (end 78.867 25.25) (width 0.25) (layer F.Cu) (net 2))
 (segment (start 36.425 30.287) (end 32.93 33.782) (width 0.25) (layer F.Cu) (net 2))
 (segment (start 38.251 30.287) (end 36.425 30.287) (width 0.25) (layer F.Cu) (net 2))
 (segment (start 32.893 39.3954) (end 32.893 42.9514) (width 0.25) (layer F.Cu) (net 27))
 (segment (start 75.40625 32.71075) (end 78.867 29.25) (width 0.25) (layer B.Cu) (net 27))
 (segment (start 75.40625 44.45) (end 75.40625 32.71075) (width 0.25) (layer B.Cu) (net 27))
 (segment (start 74.6125 45.24375) (end 75.40625 44.45) (width 0.25) (layer B.Cu) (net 27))
 (segment (start 35.18535 45.24375) (end 74.6125 45.24375) (width 0.25) (layer B.Cu) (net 27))
 (segment (start 32.893 42.9514) (end 35.18535 45.24375) (width 0.25) (layer B.Cu) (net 27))
 (segment (start 30.353 39.8526) (end 30.353 43.4086) (width 0.25) (layer F.Cu) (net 28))
 (segment (start 83.14199 30.67501) (end 83.467 30.35) (width 0.25) (layer F.Cu) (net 28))
 (segment (start 74.59201 30.67501) (end 83.14199 30.67501) (width 0.25) (layer F.Cu) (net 28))
 (segment (start 74.267 30.35) (end 74.59201 30.67501) (width 0.25) (layer F.Cu) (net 28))
 (segment (start 74.267 31.4045) (end 74.267 30.35) (width 0.25) (layer F.Cu) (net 28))
 (segment (start 75.40625 32.54375) (end 74.267 31.4045) (width 0.25) (layer F.Cu) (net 28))
 (segment (start 75.40625 44.45) (end 75.40625 32.54375) (width 0.25) (layer F.Cu) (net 28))
 (segment (start 32.18815 45.24375) (end 74.6125 45.24375) (width 0.25) (layer F.Cu) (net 28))
 (segment (start 74.6125 45.24375) (end 75.40625 44.45) (width 0.25) (layer F.Cu) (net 28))
 (segment (start 30.353 43.4086) (end 32.18815 45.24375) (width 0.25) (layer F.Cu) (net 28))
 (segment (start 50.623 24.1054) (end 50.673 24.1554) (width 0.25) (layer F.Cu) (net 16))
 (segment (start 50.623 21.0566) (end 50.623 24.1054) (width 0.25) (layer F.Cu) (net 16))
 (segment (start 58.243 24.5626) (end 58.293 24.6126) (width 0.25) (layer F.Cu) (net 19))
 (segment (start 58.243 20.5994) (end 58.243 24.5626) (width 0.25) (layer F.Cu) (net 19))
 (segment (start 45.593 21.1066) (end 45.543 21.0566) (width 0.25) (layer F.Cu) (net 14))
 (segment (start 45.593 24.1554) (end 45.593 21.1066) (width 0.25) (layer F.Cu) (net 14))
 (segment (start 55.703 24.1054) (end 55.753 24.1554) (width 0.25) (layer F.Cu) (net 18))
 (segment (start 55.703 21.0566) (end 55.703 24.1054) (width 0.25) (layer F.Cu) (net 18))
 (segment (start 48.133 20.6494) (end 48.083 20.5994) (width 0.25) (layer F.Cu) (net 15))
 (segment (start 48.133 24.6126) (end 48.133 20.6494) (width 0.25) (layer F.Cu) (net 15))
 (segment (start 53.163 24.5626) (end 53.213 24.6126) (width 0.25) (layer F.Cu) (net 17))
 (segment (start 53.163 20.5994) (end 53.163 24.5626) (width 0.25) (layer F.Cu) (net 17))
 (segment (start 43.053 24.6126) (end 43.053 20.5994) (width 0.25) (layer F.Cu) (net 13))
 (segment (start 40.513 24.1554) (end 40.513 21.0566) (width 0.25) (layer F.Cu) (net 12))
 (segment (start 37.973 24.6126) (end 37.973 20.5994) (width 0.25) (layer F.Cu) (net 4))
 (segment (start 66.675 30.607) (end 69.215 33.147) (width 0.25) (layer B.Cu) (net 4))
 (segment (start 65.405 30.607) (end 66.675 30.607) (width 0.25) (layer B.Cu) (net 4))
 (segment (start 63.627 28.829) (end 65.405 30.607) (width 0.25) (layer B.Cu) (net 4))
 (segment (start 63.627 26.543) (end 63.627 28.829) (width 0.25) (layer B.Cu) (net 4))
 (segment (start 59.817 22.733) (end 63.627 26.543) (width 0.25) (layer B.Cu) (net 4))
 (segment (start 39.8526 22.733) (end 59.817 22.733) (width 0.25) (layer B.Cu) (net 4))
 (segment (start 37.973 24.6126) (end 39.8526 22.733) (width 0.25) (layer B.Cu) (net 4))
 (segment (start 69.215 33.147) (end 71.40575 30.95625) (width 0.25) (layer F.Cu) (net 4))
 (segment (start 71.40575 30.95625) (end 71.40575 28.60675) (width 0.25) (layer F.Cu) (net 4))
 (segment (start 71.40575 28.60675) (end 77.7625 22.25) (width 0.25) (layer F.Cu) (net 4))
 (segment (start 73.279 37.211) (end 69.215 33.147) (width 0.25) (layer B.Cu) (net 4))
 (segment (start 73.279 42.418) (end 73.279 37.211) (width 0.25) (layer B.Cu) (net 4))
 (segment (start 77.7625 22.25) (end 78.867 22.25) (width 0.25) (layer F.Cu) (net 4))
 (segment (start 35.433 24.1554) (end 35.433 21.0566) (width 0.25) (layer F.Cu) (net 11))
 (segment (start 35.433 20.92325) (end 35.433 21.0566) (width 0.25) (layer F.Cu) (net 11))
 (segment (start 36.931851 19.424399) (end 35.433 20.92325) (width 0.25) (layer F.Cu) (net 11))
 (segment (start 70.993 21.844) (end 70.993 20.193) (width 0.25) (layer F.Cu) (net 11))
 (segment (start 70.224399 19.424399) (end 68.681851 19.424399) (width 0.25) (layer F.Cu) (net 11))
 (segment (start 70.993 20.193) (end 70.224399 19.424399) (width 0.25) (layer F.Cu) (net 11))
 (segment (start 68.681851 19.424399) (end 36.931851 19.424399) (width 0.25) (layer F.Cu) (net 11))
 (segment (start 68.921835 19.424399) (end 68.681851 19.424399) (width 0.25) (layer F.Cu) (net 11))
 (segment (start 65.659 42.418) (end 65.659 38.6715) (width 0.25) (layer B.Cu) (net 3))
 (segment (start 62.870199 35.882699) (end 56.520199 35.882699) (width 0.25) (layer B.Cu) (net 3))
 (segment (start 65.659 38.6715) (end 62.870199 35.882699) (width 0.25) (layer B.Cu) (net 3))
 (segment (start 56.520199 35.882699) (end 50.00625 29.36875) (width 0.25) (layer B.Cu) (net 3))
 (segment (start 41.28275 29.36875) (end 41.251 29.337) (width 0.25) (layer B.Cu) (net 3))
 (segment (start 50.00625 29.36875) (end 46.83125 29.36875) (width 0.25) (layer B.Cu) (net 3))
 (segment (start 46.83125 29.36875) (end 41.28275 29.36875) (width 0.25) (layer B.Cu) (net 3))
 (via (at 46.83125 29.36875) (size 0.8) (drill 0.4) (layers F.Cu B.Cu) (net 3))
 (segment (start 46.7995 29.337) (end 46.83125 29.36875) (width 0.25) (layer F.Cu) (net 3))
 (segment (start 41.251 29.337) (end 46.7995 29.337) (width 0.25) (layer F.Cu) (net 3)))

